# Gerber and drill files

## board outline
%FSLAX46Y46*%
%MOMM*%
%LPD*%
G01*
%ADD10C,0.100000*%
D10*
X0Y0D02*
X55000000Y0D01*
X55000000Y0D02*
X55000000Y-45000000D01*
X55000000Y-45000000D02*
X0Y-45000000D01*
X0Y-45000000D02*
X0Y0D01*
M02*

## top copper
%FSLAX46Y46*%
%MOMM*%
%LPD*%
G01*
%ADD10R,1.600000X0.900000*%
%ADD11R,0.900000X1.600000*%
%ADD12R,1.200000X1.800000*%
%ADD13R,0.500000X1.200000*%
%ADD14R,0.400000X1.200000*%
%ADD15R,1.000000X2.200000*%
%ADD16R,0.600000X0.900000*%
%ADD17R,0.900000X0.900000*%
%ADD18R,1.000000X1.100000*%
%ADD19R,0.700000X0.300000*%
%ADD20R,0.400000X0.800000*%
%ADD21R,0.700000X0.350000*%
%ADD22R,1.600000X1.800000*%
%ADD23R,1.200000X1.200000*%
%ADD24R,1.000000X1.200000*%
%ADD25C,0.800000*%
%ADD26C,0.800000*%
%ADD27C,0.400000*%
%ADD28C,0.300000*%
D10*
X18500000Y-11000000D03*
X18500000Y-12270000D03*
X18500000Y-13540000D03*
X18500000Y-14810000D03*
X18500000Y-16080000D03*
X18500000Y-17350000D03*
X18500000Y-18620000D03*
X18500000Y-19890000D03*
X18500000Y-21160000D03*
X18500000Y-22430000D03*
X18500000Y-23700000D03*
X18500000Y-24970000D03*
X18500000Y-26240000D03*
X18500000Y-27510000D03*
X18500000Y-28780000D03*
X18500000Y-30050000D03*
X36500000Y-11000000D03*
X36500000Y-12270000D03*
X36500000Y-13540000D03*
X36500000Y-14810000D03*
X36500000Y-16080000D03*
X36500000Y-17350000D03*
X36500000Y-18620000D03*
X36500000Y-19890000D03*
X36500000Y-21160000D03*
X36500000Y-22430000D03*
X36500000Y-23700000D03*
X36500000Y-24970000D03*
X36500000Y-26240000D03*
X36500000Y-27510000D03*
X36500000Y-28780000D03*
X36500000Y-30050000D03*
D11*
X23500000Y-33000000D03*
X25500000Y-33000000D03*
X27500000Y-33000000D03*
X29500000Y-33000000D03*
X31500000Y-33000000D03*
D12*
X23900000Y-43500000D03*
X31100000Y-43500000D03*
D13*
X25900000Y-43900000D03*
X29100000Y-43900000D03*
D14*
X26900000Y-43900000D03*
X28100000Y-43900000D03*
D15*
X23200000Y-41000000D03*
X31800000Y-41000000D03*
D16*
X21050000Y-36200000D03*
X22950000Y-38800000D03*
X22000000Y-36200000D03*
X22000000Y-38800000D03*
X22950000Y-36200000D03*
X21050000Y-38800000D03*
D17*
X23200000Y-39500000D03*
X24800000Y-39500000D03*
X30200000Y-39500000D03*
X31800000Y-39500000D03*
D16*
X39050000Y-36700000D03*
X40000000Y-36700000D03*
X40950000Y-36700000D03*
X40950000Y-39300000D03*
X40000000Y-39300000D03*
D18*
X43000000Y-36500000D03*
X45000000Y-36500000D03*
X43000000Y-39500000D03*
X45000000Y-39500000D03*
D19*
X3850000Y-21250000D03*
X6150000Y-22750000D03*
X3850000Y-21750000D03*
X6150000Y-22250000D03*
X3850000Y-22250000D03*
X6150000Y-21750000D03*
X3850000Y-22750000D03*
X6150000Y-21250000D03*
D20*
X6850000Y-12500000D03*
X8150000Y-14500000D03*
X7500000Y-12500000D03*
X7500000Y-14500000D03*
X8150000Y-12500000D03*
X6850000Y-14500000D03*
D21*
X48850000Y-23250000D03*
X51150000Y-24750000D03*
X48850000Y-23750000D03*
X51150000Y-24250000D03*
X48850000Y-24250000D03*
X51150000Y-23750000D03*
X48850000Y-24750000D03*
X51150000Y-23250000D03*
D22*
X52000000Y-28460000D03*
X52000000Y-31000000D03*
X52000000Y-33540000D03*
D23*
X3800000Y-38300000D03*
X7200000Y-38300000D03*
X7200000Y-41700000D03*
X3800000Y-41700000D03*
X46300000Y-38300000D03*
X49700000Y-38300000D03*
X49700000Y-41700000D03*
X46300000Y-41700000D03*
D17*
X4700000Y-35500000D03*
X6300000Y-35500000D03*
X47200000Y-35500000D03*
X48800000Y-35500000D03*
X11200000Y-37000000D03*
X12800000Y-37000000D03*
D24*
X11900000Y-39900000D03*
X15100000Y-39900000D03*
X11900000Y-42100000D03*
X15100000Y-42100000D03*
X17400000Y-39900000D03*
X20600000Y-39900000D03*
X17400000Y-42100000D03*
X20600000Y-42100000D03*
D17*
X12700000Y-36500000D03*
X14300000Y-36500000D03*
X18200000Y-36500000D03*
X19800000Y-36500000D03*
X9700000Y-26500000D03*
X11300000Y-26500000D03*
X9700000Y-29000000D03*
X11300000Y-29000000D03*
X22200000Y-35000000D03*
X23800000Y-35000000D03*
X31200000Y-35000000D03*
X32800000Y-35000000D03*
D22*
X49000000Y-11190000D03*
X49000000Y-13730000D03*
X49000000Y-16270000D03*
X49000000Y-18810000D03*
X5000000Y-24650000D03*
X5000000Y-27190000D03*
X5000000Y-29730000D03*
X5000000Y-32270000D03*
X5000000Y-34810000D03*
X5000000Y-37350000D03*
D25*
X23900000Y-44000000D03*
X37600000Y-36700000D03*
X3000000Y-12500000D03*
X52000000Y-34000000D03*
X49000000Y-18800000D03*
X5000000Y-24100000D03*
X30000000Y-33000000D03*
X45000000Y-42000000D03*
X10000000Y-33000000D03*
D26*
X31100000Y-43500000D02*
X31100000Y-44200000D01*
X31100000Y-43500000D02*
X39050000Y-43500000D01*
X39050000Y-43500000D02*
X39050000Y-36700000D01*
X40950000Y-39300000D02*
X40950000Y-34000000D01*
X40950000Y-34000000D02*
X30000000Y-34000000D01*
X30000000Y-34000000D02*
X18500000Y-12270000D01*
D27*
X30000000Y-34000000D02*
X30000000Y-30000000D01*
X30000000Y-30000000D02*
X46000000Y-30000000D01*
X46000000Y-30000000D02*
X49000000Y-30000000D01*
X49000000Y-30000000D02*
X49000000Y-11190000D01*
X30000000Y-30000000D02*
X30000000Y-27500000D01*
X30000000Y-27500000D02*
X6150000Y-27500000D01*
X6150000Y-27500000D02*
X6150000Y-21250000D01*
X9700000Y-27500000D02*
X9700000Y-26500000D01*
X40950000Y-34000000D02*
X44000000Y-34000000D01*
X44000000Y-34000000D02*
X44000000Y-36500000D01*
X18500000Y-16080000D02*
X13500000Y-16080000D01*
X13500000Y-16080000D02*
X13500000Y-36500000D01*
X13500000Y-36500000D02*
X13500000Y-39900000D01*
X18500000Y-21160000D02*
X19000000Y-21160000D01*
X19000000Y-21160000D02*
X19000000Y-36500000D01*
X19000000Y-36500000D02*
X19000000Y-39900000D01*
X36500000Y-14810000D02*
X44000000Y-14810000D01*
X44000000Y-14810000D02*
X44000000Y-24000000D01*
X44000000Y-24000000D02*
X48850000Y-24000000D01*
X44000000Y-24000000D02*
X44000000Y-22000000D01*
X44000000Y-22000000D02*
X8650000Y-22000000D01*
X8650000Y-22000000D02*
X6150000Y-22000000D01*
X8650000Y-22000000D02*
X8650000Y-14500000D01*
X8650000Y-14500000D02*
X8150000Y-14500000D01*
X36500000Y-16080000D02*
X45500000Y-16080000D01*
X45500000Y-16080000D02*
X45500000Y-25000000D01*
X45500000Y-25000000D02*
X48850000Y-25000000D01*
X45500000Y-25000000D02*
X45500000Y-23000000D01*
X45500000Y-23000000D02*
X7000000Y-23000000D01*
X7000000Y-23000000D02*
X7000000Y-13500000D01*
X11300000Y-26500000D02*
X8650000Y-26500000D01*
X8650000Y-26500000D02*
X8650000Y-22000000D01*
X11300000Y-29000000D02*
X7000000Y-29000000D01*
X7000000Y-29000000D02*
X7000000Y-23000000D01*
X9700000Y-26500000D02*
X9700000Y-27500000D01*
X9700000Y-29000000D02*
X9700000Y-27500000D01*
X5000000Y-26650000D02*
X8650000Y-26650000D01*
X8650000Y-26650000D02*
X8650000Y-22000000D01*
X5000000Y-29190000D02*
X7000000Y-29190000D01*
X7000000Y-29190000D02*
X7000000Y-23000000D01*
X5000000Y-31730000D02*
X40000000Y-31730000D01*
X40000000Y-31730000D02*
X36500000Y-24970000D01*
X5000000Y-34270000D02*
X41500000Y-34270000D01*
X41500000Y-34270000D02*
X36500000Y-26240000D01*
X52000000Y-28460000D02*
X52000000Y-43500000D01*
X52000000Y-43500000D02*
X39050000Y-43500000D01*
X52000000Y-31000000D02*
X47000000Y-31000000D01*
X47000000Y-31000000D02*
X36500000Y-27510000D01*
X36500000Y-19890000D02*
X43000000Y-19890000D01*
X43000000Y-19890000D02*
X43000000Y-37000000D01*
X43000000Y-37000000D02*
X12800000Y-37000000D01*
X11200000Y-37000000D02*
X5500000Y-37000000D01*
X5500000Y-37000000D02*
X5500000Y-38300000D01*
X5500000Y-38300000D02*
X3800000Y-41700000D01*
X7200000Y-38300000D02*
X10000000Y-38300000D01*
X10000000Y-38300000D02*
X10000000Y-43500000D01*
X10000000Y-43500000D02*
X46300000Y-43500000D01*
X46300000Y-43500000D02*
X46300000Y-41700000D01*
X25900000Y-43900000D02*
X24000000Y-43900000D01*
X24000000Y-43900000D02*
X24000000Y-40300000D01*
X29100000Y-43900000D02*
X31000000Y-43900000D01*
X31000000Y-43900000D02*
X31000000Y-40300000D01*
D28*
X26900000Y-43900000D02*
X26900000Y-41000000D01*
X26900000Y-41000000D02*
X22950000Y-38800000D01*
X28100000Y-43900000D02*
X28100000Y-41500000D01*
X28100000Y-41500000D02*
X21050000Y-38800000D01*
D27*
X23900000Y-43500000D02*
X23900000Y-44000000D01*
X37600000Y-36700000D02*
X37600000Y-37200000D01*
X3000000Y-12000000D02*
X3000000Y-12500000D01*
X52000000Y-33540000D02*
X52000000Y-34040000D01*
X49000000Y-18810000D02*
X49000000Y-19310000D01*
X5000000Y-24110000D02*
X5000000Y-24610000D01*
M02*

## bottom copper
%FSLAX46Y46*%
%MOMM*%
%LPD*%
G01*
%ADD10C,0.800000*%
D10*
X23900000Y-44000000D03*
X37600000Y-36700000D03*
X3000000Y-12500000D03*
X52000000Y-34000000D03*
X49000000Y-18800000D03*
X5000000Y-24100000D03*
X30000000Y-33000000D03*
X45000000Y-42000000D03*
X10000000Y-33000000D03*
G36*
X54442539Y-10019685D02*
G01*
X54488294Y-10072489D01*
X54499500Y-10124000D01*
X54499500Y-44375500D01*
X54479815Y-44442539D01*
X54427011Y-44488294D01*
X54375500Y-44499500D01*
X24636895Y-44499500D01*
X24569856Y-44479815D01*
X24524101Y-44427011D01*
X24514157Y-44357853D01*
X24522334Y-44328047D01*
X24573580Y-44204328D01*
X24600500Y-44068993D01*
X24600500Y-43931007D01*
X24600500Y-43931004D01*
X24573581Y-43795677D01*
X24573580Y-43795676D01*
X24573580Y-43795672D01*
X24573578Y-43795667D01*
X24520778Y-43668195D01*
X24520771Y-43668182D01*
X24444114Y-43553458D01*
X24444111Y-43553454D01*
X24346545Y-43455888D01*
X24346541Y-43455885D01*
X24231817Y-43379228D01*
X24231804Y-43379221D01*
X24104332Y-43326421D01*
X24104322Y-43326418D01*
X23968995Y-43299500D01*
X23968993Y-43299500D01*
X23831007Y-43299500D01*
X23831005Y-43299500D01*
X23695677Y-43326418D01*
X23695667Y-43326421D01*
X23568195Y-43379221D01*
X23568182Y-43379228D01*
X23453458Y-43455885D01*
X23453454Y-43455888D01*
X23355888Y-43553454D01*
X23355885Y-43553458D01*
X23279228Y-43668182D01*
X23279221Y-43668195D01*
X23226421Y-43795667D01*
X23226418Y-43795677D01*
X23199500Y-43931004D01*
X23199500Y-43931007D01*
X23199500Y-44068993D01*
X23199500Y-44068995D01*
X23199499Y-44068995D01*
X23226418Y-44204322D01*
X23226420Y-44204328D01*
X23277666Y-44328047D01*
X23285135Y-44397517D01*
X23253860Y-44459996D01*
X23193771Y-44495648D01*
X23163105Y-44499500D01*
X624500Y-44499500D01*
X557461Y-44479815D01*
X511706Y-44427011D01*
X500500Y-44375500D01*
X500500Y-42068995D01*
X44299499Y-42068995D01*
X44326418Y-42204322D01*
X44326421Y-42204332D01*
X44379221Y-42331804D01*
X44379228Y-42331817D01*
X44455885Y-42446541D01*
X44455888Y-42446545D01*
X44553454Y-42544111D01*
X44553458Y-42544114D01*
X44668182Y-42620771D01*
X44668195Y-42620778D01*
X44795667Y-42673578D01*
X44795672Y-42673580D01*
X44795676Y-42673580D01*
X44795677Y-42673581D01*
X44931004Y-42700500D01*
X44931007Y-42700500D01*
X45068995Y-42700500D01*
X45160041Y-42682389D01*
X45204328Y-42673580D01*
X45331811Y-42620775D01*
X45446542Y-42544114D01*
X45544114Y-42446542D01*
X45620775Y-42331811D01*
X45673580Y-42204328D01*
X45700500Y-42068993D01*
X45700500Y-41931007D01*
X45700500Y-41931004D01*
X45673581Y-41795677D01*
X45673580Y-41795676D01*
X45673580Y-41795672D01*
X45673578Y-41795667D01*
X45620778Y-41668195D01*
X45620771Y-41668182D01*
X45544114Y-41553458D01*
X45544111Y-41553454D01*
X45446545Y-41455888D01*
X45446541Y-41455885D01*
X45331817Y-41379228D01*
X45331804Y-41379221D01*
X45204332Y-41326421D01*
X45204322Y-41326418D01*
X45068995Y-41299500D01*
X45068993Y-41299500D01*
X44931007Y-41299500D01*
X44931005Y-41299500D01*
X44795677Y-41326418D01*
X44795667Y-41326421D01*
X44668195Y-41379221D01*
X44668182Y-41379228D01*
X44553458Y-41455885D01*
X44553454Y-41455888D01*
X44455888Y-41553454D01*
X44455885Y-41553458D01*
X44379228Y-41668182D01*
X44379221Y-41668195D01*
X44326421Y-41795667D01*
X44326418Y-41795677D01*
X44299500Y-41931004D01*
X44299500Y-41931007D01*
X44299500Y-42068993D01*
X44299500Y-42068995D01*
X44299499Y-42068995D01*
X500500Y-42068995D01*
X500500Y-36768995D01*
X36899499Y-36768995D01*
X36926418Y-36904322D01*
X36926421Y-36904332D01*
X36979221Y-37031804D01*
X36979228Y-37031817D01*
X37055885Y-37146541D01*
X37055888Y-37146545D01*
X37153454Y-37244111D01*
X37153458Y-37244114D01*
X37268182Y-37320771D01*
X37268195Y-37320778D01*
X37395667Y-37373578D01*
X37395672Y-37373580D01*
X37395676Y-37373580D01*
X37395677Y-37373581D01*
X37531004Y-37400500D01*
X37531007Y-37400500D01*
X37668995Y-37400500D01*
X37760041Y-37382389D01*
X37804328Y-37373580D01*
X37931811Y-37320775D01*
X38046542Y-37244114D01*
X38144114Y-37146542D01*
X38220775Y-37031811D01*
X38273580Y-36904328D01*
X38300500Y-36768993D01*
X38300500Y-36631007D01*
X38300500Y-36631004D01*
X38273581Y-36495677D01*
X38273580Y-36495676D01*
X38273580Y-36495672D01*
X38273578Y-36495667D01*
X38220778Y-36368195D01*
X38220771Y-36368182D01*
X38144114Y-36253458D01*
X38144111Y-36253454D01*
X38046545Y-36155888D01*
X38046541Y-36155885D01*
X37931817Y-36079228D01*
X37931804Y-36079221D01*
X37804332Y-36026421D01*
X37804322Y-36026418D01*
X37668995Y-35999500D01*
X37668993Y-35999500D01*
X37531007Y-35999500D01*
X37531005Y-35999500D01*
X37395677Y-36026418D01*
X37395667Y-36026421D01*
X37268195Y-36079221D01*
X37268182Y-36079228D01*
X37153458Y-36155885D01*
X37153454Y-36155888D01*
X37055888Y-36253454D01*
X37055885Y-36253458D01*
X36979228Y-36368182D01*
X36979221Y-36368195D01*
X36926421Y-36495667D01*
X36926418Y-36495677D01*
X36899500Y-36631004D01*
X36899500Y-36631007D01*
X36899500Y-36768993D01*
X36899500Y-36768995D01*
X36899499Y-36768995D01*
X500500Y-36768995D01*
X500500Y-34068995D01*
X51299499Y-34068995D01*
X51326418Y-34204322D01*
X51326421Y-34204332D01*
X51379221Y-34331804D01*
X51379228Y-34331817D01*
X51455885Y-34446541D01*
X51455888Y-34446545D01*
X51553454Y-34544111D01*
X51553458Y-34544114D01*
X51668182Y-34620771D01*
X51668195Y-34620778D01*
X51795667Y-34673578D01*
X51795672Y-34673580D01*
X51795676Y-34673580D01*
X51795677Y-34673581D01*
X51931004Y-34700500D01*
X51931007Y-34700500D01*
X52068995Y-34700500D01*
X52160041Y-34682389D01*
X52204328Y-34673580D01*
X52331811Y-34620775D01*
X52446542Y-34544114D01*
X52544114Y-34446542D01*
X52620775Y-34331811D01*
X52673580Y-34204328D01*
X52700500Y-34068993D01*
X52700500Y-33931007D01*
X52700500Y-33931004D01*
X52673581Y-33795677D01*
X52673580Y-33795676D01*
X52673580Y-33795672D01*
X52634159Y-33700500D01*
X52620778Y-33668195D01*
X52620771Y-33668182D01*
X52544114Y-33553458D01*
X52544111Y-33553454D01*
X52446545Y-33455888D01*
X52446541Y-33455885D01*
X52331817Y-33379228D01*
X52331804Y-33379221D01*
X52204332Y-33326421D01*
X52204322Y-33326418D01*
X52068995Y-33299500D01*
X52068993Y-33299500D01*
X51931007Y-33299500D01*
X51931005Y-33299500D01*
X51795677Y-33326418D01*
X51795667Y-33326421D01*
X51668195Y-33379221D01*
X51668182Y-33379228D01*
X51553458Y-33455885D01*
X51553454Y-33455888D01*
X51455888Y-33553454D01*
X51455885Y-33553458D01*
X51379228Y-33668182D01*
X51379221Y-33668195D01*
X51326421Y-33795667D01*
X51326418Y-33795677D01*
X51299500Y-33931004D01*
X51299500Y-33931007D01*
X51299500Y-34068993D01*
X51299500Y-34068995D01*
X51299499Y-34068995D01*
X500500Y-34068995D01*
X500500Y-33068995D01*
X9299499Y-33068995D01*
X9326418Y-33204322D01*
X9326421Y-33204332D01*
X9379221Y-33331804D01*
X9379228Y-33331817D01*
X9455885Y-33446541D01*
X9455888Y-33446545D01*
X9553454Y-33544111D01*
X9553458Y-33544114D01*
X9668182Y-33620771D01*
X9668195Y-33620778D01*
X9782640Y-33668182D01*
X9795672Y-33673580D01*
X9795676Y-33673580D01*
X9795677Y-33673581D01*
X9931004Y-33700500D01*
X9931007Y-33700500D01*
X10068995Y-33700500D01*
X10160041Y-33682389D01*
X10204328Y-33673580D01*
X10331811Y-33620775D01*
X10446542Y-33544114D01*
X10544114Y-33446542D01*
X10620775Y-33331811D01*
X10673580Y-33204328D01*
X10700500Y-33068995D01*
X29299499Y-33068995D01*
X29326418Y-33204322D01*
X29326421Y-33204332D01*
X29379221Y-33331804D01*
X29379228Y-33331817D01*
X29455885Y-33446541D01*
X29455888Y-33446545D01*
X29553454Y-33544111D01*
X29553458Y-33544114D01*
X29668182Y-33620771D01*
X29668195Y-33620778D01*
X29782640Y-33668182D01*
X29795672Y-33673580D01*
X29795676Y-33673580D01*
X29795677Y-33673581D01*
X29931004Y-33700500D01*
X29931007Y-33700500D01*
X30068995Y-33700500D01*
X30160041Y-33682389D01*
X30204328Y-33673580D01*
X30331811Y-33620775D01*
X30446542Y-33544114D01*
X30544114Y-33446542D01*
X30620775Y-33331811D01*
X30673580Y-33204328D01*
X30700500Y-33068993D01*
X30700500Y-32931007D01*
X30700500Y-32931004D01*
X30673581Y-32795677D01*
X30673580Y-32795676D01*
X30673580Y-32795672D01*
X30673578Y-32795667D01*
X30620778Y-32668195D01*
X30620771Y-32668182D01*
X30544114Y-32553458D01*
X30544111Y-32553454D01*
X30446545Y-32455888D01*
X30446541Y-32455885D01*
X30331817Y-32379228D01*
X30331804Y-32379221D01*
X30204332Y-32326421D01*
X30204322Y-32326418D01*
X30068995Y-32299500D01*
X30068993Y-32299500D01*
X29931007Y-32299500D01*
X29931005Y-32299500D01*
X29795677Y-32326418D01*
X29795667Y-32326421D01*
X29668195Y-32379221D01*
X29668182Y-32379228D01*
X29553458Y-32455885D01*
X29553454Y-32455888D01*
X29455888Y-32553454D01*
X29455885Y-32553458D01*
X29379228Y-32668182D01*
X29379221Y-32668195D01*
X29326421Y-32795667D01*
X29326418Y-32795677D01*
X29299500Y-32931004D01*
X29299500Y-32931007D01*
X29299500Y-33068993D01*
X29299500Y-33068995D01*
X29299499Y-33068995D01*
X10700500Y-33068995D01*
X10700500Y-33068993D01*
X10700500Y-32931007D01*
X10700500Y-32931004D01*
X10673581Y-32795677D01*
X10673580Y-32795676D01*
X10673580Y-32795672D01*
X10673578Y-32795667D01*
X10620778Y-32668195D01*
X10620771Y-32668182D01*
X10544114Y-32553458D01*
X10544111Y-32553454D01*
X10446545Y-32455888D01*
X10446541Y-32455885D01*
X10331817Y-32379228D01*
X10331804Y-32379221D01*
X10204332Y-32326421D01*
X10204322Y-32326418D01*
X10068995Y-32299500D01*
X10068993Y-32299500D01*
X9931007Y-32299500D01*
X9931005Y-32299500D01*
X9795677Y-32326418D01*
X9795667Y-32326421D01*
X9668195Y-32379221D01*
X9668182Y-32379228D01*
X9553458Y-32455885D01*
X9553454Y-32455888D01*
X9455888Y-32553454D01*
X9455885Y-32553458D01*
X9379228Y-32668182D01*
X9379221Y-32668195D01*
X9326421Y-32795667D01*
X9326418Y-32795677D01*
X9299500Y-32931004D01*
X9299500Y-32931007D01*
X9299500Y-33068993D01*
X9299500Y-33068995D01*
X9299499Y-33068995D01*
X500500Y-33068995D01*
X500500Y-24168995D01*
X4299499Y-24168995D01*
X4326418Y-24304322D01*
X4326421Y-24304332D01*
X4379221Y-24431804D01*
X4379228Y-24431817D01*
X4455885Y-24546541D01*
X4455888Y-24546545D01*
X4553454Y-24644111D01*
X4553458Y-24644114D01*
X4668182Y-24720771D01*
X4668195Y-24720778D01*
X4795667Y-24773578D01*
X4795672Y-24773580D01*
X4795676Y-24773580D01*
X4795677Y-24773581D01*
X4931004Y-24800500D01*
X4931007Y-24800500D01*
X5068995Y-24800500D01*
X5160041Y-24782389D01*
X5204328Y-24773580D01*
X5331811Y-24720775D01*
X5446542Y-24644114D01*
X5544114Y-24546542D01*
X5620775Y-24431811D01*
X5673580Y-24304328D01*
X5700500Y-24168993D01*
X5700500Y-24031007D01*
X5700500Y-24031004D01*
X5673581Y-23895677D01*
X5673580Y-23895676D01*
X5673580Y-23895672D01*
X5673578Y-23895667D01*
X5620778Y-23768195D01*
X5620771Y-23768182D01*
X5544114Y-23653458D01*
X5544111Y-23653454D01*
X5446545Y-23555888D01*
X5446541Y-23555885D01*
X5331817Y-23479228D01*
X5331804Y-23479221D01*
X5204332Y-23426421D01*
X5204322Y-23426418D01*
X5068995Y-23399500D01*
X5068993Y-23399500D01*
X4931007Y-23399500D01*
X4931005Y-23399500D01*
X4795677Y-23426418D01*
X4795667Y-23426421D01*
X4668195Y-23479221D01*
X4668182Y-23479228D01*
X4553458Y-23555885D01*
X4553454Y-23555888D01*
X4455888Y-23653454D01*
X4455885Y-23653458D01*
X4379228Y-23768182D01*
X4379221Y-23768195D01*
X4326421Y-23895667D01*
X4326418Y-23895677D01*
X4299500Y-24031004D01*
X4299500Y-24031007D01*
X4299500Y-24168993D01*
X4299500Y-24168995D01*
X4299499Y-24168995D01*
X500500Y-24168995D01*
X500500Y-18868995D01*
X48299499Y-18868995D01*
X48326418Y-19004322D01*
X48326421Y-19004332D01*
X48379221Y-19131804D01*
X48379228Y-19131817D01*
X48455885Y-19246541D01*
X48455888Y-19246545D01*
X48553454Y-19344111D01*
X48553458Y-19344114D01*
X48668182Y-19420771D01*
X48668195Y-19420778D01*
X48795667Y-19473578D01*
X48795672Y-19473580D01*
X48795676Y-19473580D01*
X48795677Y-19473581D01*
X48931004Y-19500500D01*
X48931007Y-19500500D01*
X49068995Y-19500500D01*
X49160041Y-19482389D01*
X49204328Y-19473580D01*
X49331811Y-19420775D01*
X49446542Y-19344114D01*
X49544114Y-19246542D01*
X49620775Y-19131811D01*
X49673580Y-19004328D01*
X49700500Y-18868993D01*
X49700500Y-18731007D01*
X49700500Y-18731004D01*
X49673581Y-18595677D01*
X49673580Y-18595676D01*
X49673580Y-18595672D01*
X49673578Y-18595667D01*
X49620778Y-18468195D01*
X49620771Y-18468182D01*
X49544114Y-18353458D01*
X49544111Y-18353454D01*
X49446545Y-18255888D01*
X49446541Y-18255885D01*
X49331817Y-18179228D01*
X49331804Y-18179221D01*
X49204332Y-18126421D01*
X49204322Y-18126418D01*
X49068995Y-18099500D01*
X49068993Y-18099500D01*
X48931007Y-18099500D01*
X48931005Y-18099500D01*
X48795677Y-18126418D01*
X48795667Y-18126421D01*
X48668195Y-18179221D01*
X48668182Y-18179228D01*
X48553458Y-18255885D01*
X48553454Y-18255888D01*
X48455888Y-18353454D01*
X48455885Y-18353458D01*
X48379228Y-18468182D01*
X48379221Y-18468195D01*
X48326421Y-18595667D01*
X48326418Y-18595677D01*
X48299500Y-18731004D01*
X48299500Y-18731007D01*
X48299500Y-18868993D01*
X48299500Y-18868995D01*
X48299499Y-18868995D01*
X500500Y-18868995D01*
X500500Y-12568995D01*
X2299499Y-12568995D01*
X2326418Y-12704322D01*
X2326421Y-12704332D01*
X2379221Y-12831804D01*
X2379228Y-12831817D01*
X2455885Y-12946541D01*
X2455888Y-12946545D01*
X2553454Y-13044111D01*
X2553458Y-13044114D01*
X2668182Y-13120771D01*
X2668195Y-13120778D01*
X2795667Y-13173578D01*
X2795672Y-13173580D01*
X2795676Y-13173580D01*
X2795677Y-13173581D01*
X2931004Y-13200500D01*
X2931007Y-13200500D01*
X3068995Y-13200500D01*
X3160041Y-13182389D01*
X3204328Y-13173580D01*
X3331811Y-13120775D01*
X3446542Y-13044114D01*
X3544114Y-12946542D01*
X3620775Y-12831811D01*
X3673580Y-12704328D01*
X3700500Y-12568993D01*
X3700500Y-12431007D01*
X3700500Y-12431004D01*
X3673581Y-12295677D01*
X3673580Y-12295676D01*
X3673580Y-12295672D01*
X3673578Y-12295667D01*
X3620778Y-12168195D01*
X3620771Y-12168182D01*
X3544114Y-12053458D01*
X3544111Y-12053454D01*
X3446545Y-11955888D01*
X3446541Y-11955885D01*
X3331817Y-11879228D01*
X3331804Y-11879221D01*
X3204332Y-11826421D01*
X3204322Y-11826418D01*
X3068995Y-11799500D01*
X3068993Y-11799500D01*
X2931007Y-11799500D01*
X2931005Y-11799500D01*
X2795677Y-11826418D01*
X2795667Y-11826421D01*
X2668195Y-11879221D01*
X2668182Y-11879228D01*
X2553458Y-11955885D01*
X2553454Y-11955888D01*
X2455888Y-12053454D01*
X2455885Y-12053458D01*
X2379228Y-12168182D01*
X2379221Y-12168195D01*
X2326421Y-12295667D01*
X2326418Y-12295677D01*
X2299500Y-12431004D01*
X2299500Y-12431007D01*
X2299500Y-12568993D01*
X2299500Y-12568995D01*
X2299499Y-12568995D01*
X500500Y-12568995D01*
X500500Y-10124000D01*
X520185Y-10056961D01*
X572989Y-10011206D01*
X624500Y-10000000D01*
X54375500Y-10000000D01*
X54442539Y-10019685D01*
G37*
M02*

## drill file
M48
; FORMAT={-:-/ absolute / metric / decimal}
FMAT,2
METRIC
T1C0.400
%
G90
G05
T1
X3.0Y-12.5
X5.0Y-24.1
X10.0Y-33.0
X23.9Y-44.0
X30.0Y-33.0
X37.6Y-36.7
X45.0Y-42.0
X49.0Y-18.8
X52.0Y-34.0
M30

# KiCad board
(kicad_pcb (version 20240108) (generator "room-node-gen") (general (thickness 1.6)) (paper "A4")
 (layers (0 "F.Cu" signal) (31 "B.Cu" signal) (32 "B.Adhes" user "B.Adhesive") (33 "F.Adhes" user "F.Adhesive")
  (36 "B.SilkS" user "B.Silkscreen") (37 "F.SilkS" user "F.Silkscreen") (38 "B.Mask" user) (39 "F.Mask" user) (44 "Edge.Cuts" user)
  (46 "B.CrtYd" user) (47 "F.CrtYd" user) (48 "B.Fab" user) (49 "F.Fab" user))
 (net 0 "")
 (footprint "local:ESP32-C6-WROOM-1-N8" (layer "F.Cu") (at 27.500 22.000 0)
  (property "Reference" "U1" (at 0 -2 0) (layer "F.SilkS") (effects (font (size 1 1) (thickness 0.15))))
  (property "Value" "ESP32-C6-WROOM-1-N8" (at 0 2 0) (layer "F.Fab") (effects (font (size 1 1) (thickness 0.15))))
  (pad "1" smd rect (at -9.000 -11.000) (size 1.600 0.900) (layers "F.Cu"))
  (pad "2" smd rect (at -9.000 -9.730) (size 1.600 0.900) (layers "F.Cu"))
  (pad "3" smd rect (at -9.000 -8.460) (size 1.600 0.900) (layers "F.Cu"))
  (pad "4" smd rect (at -9.000 -7.190) (size 1.600 0.900) (layers "F.Cu"))
  (pad "5" smd rect (at -9.000 -5.920) (size 1.600 0.900) (layers "F.Cu"))
  (pad "6" smd rect (at -9.000 -4.650) (size 1.600 0.900) (layers "F.Cu"))
  (pad "7" smd rect (at -9.000 -3.380) (size 1.600 0.900) (layers "F.Cu"))
  (pad "8" smd rect (at -9.000 -2.110) (size 1.600 0.900) (layers "F.Cu"))
  (pad "9" smd rect (at -9.000 -0.840) (size 1.600 0.900) (layers "F.Cu"))
  (pad "10" smd rect (at -9.000 0.430) (size 1.600 0.900) (layers "F.Cu"))
  (pad "11" smd rect (at -9.000 1.700) (size 1.600 0.900) (layers "F.Cu"))
  (pad "12" smd rect (at -9.000 2.970) (size 1.600 0.900) (layers "F.Cu"))
  (pad "13" smd rect (at -9.000 4.240) (size 1.600 0.900) (layers "F.Cu"))
  (pad "14" smd rect (at -9.000 5.510) (size 1.600 0.900) (layers "F.Cu"))
  (pad "15" smd rect (at -9.000 6.780) (size 1.600 0.900) (layers "F.Cu"))
  (pad "16" smd rect (at -9.000 8.050) (size 1.600 0.900) (layers "F.Cu"))
  (pad "17" smd rect (at 9.000 -11.000) (size 1.600 0.900) (layers "F.Cu"))
  (pad "18" smd rect (at 9.000 -9.730) (size 1.600 0.900) (layers "F.Cu"))
  (pad "19" smd rect (at 9.000 -8.460) (size 1.600 0.900) (layers "F.Cu"))
  (pad "20" smd rect (at 9.000 -7.190) (size 1.600 0.900) (layers "F.Cu"))
  (pad "21" smd rect (at 9.000 -5.920) (size 1.600 0.900) (layers "F.Cu"))
  (pad "22" smd rect (at 9.000 -4.650) (size 1.600 0.900) (layers "F.Cu"))
  (pad "23" smd rect (at 9.000 -3.380) (size 1.600 0.900) (layers "F.Cu"))
  (pad "24" smd rect (at 9.000 -2.110) (size 1.600 0.900) (layers "F.Cu"))
  (pad "25" smd rect (at 9.000 -0.840) (size 1.600 0.900) (layers "F.Cu"))
  (pad "26" smd rect (at 9.000 0.430) (size 1.600 0.900) (layers "F.Cu"))
  (pad "27" smd rect (at 9.000 1.700) (size 1.600 0.900) (layers "F.Cu"))
  (pad "28" smd rect (at 9.000 2.970) (size 1.600 0.900) (layers "F.Cu"))
  (pad "29" smd rect (at 9.000 4.240) (size 1.600 0.900) (layers "F.Cu"))
  (pad "30" smd rect (at 9.000 5.510) (size 1.600 0.900) (layers "F.Cu"))
  (pad "31" smd rect (at 9.000 6.780) (size 1.600 0.900) (layers "F.Cu"))
  (pad "32" smd rect (at 9.000 8.050) (size 1.600 0.900) (layers "F.Cu"))
  (pad "33" smd rect (at -4.000 11.000) (size 0.900 1.600) (layers "F.Cu"))
  (pad "34" smd rect (at -2.000 11.000) (size 0.900 1.600) (layers "F.Cu"))
  (pad "35" smd rect (at 0.000 11.000) (size 0.900 1.600) (layers "F.Cu"))
  (pad "36" smd rect (at 2.000 11.000) (size 0.900 1.600) (layers "F.Cu"))
  (pad "37" smd rect (at 4.000 11.000) (size 0.900 1.600) (layers "F.Cu")))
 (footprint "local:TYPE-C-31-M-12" (layer "F.Cu") (at 27.500 42.000 0)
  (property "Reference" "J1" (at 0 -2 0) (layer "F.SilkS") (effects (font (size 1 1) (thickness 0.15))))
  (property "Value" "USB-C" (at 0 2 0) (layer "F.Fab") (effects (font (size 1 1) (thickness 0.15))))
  (pad "GND" smd rect (at -3.600 1.500) (size 1.200 1.800) (layers "F.Cu"))
  (pad "VBUS" smd rect (at 3.600 1.500) (size 1.200 1.800) (layers "F.Cu"))
  (pad "CC1" smd rect (at -1.600 1.900) (size 0.500 1.200) (layers "F.Cu"))
  (pad "CC2" smd rect (at 1.600 1.900) (size 0.500 1.200) (layers "F.Cu"))
  (pad "DM" smd rect (at -0.600 1.900) (size 0.400 1.200) (layers "F.Cu"))
  (pad "DP" smd rect (at 0.600 1.900) (size 0.400 1.200) (layers "F.Cu"))
  (pad "SH1" smd rect (at -4.300 -1.000) (size 1.000 2.200) (layers "F.Cu"))
  (pad "SH2" smd rect (at 4.300 -1.000) (size 1.000 2.200) (layers "F.Cu")))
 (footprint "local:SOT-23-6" (layer "F.Cu") (at 22.000 37.500 0)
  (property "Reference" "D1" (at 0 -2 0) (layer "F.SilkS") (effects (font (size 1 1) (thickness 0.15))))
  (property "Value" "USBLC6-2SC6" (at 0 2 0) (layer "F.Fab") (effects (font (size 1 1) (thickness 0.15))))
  (pad "1" smd rect (at -0.950 -1.300) (size 0.600 0.900) (layers "F.Cu"))
  (pad "4" smd rect (at 0.950 1.300) (size 0.600 0.900) (layers "F.Cu"))
  (pad "2" smd rect (at 0.000 -1.300) (size 0.600 0.900) (layers "F.Cu"))
  (pad "5" smd rect (at 0.000 1.300) (size 0.600 0.900) (layers "F.Cu"))
  (pad "3" smd rect (at 0.950 -1.300) (size 0.600 0.900) (layers "F.Cu"))
  (pad "6" smd rect (at -0.950 1.300) (size 0.600 0.900) (layers "F.Cu")))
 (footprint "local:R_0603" (layer "F.Cu") (at 24.000 39.500 0)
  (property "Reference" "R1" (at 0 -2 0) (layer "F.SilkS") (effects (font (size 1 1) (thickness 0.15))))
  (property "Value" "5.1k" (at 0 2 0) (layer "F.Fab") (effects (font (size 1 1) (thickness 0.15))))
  (pad "1" smd rect (at -0.800 0.000) (size 0.900 0.900) (layers "F.Cu"))
  (pad "2" smd rect (at 0.800 0.000) (size 0.900 0.900) (layers "F.Cu")))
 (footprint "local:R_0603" (layer "F.Cu") (at 31.000 39.500 0)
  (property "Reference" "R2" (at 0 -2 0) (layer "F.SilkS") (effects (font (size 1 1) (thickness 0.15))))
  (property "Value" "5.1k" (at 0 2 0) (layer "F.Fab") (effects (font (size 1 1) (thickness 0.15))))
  (pad "1" smd rect (at -0.800 0.000) (size 0.900 0.900) (layers "F.Cu"))
  (pad "2" smd rect (at 0.800 0.000) (size 0.900 0.900) (layers "F.Cu")))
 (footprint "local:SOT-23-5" (layer "F.Cu") (at 40.000 38.000 0)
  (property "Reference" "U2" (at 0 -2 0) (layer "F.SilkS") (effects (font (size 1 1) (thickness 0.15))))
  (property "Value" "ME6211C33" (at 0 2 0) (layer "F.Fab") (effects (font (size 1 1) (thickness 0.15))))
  (pad "1" smd rect (at -0.950 -1.300) (size 0.600 0.900) (layers "F.Cu"))
  (pad "2" smd rect (at 0.000 -1.300) (size 0.600 0.900) (layers "F.Cu"))
  (pad "3" smd rect (at 0.950 -1.300) (size 0.600 0.900) (layers "F.Cu"))
  (pad "4" smd rect (at 0.950 1.300) (size 0.600 0.900) (layers "F.Cu"))
  (pad "5" smd rect (at 0.000 1.300) (size 0.600 0.900) (layers "F.Cu")))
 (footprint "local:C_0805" (layer "F.Cu") (at 44.000 36.500 0)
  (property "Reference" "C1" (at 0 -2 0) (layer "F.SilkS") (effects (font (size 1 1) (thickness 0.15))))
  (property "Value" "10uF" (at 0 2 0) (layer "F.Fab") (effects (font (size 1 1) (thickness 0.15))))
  (pad "1" smd rect (at -1.000 0.000) (size 1.000 1.100) (layers "F.Cu"))
  (pad "2" smd rect (at 1.000 0.000) (size 1.000 1.100) (layers "F.Cu")))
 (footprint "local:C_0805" (layer "F.Cu") (at 44.000 39.500 0)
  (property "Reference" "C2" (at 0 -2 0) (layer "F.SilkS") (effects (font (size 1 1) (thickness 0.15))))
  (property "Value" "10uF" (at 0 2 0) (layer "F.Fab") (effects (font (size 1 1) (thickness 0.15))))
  (pad "1" smd rect (at -1.000 0.000) (size 1.000 1.100) (layers "F.Cu"))
  (pad "2" smd rect (at 1.000 0.000) (size 1.000 1.100) (layers "F.Cu")))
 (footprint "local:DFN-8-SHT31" (layer "F.Cu") (at 5.000 22.000 0)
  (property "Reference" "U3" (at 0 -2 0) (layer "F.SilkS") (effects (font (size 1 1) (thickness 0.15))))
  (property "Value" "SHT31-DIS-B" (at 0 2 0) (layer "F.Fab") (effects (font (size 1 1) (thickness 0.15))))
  (pad "1" smd rect (at -1.150 -0.750) (size 0.700 0.300) (layers "F.Cu"))
  (pad "5" smd rect (at 1.150 0.750) (size 0.700 0.300) (layers "F.Cu"))
  (pad "2" smd rect (at -1.150 -0.250) (size 0.700 0.300) (layers "F.Cu"))
  (pad "6" smd rect (at 1.150 0.250) (size 0.700 0.300) (layers "F.Cu"))
  (pad "3" smd rect (at -1.150 0.250) (size 0.700 0.300) (layers "F.Cu"))
  (pad "7" smd rect (at 1.150 -0.250) (size 0.700 0.300) (layers "F.Cu"))
  (pad "4" smd rect (at -1.150 0.750) (size 0.700 0.300) (layers "F.Cu"))
  (pad "8" smd rect (at 1.150 -0.750) (size 0.700 0.300) (layers "F.Cu")))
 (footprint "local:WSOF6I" (layer "F.Cu") (at 7.500 13.500 0)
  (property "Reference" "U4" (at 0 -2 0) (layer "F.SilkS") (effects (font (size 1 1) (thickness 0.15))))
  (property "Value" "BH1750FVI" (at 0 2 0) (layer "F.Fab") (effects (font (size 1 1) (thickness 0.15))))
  (pad "1" smd rect (at -0.650 -1.000) (size 0.400 0.800) (layers "F.Cu"))
  (pad "4" smd rect (at 0.650 1.000) (size 0.400 0.800) (layers "F.Cu"))
  (pad "2" smd rect (at 0.000 -1.000) (size 0.400 0.800) (layers "F.Cu"))
  (pad "5" smd rect (at 0.000 1.000) (size 0.400 0.800) (layers "F.Cu"))
  (pad "3" smd rect (at 0.650 -1.000) (size 0.400 0.800) (layers "F.Cu"))
  (pad "6" smd rect (at -0.650 1.000) (size 0.400 0.800) (layers "F.Cu")))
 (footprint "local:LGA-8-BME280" (layer "F.Cu") (at 50.000 24.000 0)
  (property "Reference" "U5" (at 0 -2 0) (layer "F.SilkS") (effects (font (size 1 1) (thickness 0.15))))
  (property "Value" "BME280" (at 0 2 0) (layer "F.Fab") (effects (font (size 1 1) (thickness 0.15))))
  (pad "1" smd rect (at -1.150 -0.750) (size 0.700 0.350) (layers "F.Cu"))
  (pad "5" smd rect (at 1.150 0.750) (size 0.700 0.350) (layers "F.Cu"))
  (pad "2" smd rect (at -1.150 -0.250) (size 0.700 0.350) (layers "F.Cu"))
  (pad "6" smd rect (at 1.150 0.250) (size 0.700 0.350) (layers "F.Cu"))
  (pad "3" smd rect (at -1.150 0.250) (size 0.700 0.350) (layers "F.Cu"))
  (pad "7" smd rect (at 1.150 -0.250) (size 0.700 0.350) (layers "F.Cu"))
  (pad "4" smd rect (at -1.150 0.750) (size 0.700 0.350) (layers "F.Cu"))
  (pad "8" smd rect (at 1.150 -0.750) (size 0.700 0.350) (layers "F.Cu")))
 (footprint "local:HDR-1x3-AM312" (layer "F.Cu") (at 52.000 31.000 0)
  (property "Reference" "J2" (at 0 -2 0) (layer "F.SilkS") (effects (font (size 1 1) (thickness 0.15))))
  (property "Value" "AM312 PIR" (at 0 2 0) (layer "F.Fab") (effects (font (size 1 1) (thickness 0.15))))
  (pad "VIN" smd rect (at 0.000 -2.540) (size 1.600 1.800) (layers "F.Cu"))
  (pad "OUT" smd rect (at 0.000 0.000) (size 1.600 1.800) (layers "F.Cu"))
  (pad "GND" smd rect (at 0.000 2.540) (size 1.600 1.800) (layers "F.Cu")))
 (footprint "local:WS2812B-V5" (layer "F.Cu") (at 5.500 40.000 0)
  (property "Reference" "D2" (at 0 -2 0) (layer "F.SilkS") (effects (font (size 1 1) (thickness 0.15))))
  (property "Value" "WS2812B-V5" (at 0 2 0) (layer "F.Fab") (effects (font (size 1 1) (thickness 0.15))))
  (pad "VDD" smd rect (at -1.700 -1.700) (size 1.200 1.200) (layers "F.Cu"))
  (pad "DOUT" smd rect (at 1.700 -1.700) (size 1.200 1.200) (layers "F.Cu"))
  (pad "VSS" smd rect (at 1.700 1.700) (size 1.200 1.200) (layers "F.Cu"))
  (pad "DIN" smd rect (at -1.700 1.700) (size 1.200 1.200) (layers "F.Cu")))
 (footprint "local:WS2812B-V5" (layer "F.Cu") (at 48.000 40.000 0)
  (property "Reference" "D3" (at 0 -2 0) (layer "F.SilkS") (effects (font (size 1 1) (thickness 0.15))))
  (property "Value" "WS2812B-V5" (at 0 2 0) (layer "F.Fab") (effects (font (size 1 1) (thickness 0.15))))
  (pad "VDD" smd rect (at -1.700 -1.700) (size 1.200 1.200) (layers "F.Cu"))
  (pad "DOUT" smd rect (at 1.700 -1.700) (size 1.200 1.200) (layers "F.Cu"))
  (pad "VSS" smd rect (at 1.700 1.700) (size 1.200 1.200) (layers "F.Cu"))
  (pad "DIN" smd rect (at -1.700 1.700) (size 1.200 1.200) (layers "F.Cu")))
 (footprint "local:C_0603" (layer "F.Cu") (at 5.500 35.500 0)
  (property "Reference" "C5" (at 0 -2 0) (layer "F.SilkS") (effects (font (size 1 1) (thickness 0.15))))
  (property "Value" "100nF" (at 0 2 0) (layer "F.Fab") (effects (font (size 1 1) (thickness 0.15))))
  (pad "1" smd rect (at -0.800 0.000) (size 0.900 0.900) (layers "F.Cu"))
  (pad "2" smd rect (at 0.800 0.000) (size 0.900 0.900) (layers "F.Cu")))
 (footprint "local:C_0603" (layer "F.Cu") (at 48.000 35.500 0)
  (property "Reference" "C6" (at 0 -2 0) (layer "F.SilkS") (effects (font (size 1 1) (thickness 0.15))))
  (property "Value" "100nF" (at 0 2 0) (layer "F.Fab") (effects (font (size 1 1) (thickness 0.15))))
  (pad "1" smd rect (at -0.800 0.000) (size 0.900 0.900) (layers "F.Cu"))
  (pad "2" smd rect (at 0.800 0.000) (size 0.900 0.900) (layers "F.Cu")))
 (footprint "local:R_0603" (layer "F.Cu") (at 12.000 37.000 0)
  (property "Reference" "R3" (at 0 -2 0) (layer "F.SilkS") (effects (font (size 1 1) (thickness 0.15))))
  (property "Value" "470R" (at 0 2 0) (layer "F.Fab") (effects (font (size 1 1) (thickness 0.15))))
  (pad "1" smd rect (at -0.800 0.000) (size 0.900 0.900) (layers "F.Cu"))
  (pad "2" smd rect (at 0.800 0.000) (size 0.900 0.900) (layers "F.Cu")))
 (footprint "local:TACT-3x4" (layer "F.Cu") (at 13.500 41.000 0)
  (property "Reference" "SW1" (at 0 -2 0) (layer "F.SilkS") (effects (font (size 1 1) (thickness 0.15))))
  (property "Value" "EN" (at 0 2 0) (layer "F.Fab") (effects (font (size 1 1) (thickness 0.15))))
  (pad "1" smd rect (at -1.600 -1.100) (size 1.000 1.200) (layers "F.Cu"))
  (pad "2" smd rect (at 1.600 -1.100) (size 1.000 1.200) (layers "F.Cu"))
  (pad "3" smd rect (at -1.600 1.100) (size 1.000 1.200) (layers "F.Cu"))
  (pad "4" smd rect (at 1.600 1.100) (size 1.000 1.200) (layers "F.Cu")))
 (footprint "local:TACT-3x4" (layer "F.Cu") (at 19.000 41.000 0)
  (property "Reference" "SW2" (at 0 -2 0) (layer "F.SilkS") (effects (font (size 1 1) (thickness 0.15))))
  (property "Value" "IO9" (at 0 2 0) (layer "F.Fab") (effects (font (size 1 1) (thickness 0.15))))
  (pad "1" smd rect (at -1.600 -1.100) (size 1.000 1.200) (layers "F.Cu"))
  (pad "2" smd rect (at 1.600 -1.100) (size 1.000 1.200) (layers "F.Cu"))
  (pad "3" smd rect (at -1.600 1.100) (size 1.000 1.200) (layers "F.Cu"))
  (pad "4" smd rect (at 1.600 1.100) (size 1.000 1.200) (layers "F.Cu")))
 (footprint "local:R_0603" (layer "F.Cu") (at 13.500 36.500 0)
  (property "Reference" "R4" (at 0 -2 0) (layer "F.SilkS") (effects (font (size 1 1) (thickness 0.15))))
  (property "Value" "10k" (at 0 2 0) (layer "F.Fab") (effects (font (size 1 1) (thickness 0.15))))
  (pad "1" smd rect (at -0.800 0.000) (size 0.900 0.900) (layers "F.Cu"))
  (pad "2" smd rect (at 0.800 0.000) (size 0.900 0.900) (layers "F.Cu")))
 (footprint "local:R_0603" (layer "F.Cu") (at 19.000 36.500 0)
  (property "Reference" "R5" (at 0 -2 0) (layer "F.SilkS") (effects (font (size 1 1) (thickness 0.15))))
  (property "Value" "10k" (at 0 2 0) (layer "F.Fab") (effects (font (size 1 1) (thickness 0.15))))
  (pad "1" smd rect (at -0.800 0.000) (size 0.900 0.900) (layers "F.Cu"))
  (pad "2" smd rect (at 0.800 0.000) (size 0.900 0.900) (layers "F.Cu")))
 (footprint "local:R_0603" (layer "F.Cu") (at 10.500 26.500 0)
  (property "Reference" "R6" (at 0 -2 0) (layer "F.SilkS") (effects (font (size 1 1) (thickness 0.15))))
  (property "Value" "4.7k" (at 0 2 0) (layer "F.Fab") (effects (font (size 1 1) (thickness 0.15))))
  (pad "1" smd rect (at -0.800 0.000) (size 0.900 0.900) (layers "F.Cu"))
  (pad "2" smd rect (at 0.800 0.000) (size 0.900 0.900) (layers "F.Cu")))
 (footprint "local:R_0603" (layer "F.Cu") (at 10.500 29.000 0)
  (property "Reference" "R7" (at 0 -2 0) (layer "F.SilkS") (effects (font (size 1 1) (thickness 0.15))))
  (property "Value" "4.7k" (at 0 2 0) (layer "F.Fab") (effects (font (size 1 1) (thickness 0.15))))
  (pad "1" smd rect (at -0.800 0.000) (size 0.900 0.900) (layers "F.Cu"))
  (pad "2" smd rect (at 0.800 0.000) (size 0.900 0.900) (layers "F.Cu")))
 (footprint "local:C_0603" (layer "F.Cu") (at 23.000 35.000 0)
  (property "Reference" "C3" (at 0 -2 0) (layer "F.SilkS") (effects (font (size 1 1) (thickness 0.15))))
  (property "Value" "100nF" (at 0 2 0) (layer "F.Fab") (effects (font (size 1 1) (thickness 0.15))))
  (pad "1" smd rect (at -0.800 0.000) (size 0.900 0.900) (layers "F.Cu"))
  (pad "2" smd rect (at 0.800 0.000) (size 0.900 0.900) (layers "F.Cu")))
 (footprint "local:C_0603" (layer "F.Cu") (at 32.000 35.000 0)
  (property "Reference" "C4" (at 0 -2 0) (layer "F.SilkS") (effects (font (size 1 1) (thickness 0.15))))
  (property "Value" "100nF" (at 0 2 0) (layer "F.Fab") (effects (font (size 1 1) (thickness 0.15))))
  (pad "1" smd rect (at -0.800 0.000) (size 0.900 0.900) (layers "F.Cu"))
  (pad "2" smd rect (at 0.800 0.000) (size 0.900 0.900) (layers "F.Cu")))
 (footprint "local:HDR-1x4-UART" (layer "F.Cu") (at 49.000 15.000 0)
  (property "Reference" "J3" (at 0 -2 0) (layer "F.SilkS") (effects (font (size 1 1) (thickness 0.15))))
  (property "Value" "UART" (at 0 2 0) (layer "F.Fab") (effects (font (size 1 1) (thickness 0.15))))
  (pad "3V3" smd rect (at 0.000 -3.810) (size 1.600 1.800) (layers "F.Cu"))
  (pad "TX" smd rect (at 0.000 -1.270) (size 1.600 1.800) (layers "F.Cu"))
  (pad "RX" smd rect (at 0.000 1.270) (size 1.600 1.800) (layers "F.Cu"))
  (pad "GND" smd rect (at 0.000 3.810) (size 1.600 1.800) (layers "F.Cu")))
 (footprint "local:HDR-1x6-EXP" (layer "F.Cu") (at 5.000 31.000 0)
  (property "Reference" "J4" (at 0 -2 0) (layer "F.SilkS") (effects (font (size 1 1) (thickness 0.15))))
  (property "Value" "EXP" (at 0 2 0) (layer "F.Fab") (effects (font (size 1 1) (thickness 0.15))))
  (pad "3V3" smd rect (at 0.000 -6.350) (size 1.600 1.800) (layers "F.Cu"))
  (pad "GND" smd rect (at 0.000 -3.810) (size 1.600 1.800) (layers "F.Cu"))
  (pad "SDA" smd rect (at 0.000 -1.270) (size 1.600 1.800) (layers "F.Cu"))
  (pad "SCL" smd rect (at 0.000 1.270) (size 1.600 1.800) (layers "F.Cu"))
  (pad "IO20" smd rect (at 0.000 3.810) (size 1.600 1.800) (layers "F.Cu"))
  (pad "IO21" smd rect (at 0.000 6.350) (size 1.600 1.800) (layers "F.Cu")))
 (gr_line (start 0.000 0.000) (end 55.000 0.000) (stroke (width 0.1) (type solid)) (layer "Edge.Cuts"))
 (gr_line (start 55.000 0.000) (end 55.000 45.000) (stroke (width 0.1) (type solid)) (layer "Edge.Cuts"))
 (gr_line (start 55.000 45.000) (end 0.000 45.000) (stroke (width 0.1) (type solid)) (layer "Edge.Cuts"))
 (gr_line (start 0.000 45.000) (end 0.000 0.000) (stroke (width 0.1) (type solid)) (layer "Edge.Cuts"))
 (segment (start 31.100 43.500) (end 31.100 44.200) (width 0.8) (layer "F.Cu") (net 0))
 (segment (start 31.100 43.500) (end 39.050 43.500) (width 0.8) (layer "F.Cu") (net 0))
 (segment (start 39.050 43.500) (end 39.050 36.700) (width 0.8) (layer "F.Cu") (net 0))
 (segment (start 40.950 39.300) (end 40.950 34.000) (width 0.8) (layer "F.Cu") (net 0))
 (segment (start 40.950 34.000) (end 30.000 34.000) (width 0.8) (layer "F.Cu") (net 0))
 (segment (start 30.000 34.000) (end 18.500 12.270) (width 0.8) (layer "F.Cu") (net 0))
 (segment (start 30.000 34.000) (end 30.000 30.000) (width 0.4) (layer "F.Cu") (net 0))
 (segment (start 30.000 30.000) (end 46.000 30.000) (width 0.4) (layer "F.Cu") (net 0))
 (segment (start 46.000 30.000) (end 49.000 30.000) (width 0.4) (layer "F.Cu") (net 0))
 (segment (start 49.000 30.000) (end 49.000 11.190) (width 0.4) (layer "F.Cu") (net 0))
 (segment (start 30.000 30.000) (end 30.000 27.500) (width 0.4) (layer "F.Cu") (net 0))
 (segment (start 30.000 27.500) (end 6.150 27.500) (width 0.4) (layer "F.Cu") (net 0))
 (segment (start 6.150 27.500) (end 6.150 21.250) (width 0.4) (layer "F.Cu") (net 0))
 (segment (start 9.700 27.500) (end 9.700 26.500) (width 0.4) (layer "F.Cu") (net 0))
 (segment (start 40.950 34.000) (end 44.000 34.000) (width 0.4) (layer "F.Cu") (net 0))
 (segment (start 44.000 34.000) (end 44.000 36.500) (width 0.4) (layer "F.Cu") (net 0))
 (segment (start 18.500 16.080) (end 13.500 16.080) (width 0.4) (layer "F.Cu") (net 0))
 (segment (start 13.500 16.080) (end 13.500 36.500) (width 0.4) (layer "F.Cu") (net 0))
 (segment (start 13.500 36.500) (end 13.500 39.900) (width 0.4) (layer "F.Cu") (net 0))
 (segment (start 18.500 21.160) (end 19.000 21.160) (width 0.4) (layer "F.Cu") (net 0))
 (segment (start 19.000 21.160) (end 19.000 36.500) (width 0.4) (layer "F.Cu") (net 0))
 (segment (start 19.000 36.500) (end 19.000 39.900) (width 0.4) (layer "F.Cu") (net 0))
 (segment (start 36.500 14.810) (end 44.000 14.810) (width 0.4) (layer "F.Cu") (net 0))
 (segment (start 44.000 14.810) (end 44.000 24.000) (width 0.4) (layer "F.Cu") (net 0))
 (segment (start 44.000 24.000) (end 48.850 24.000) (width 0.4) (layer "F.Cu") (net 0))
 (segment (start 44.000 24.000) (end 44.000 22.000) (width 0.4) (layer "F.Cu") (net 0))
 (segment (start 44.000 22.000) (end 8.650 22.000) (width 0.4) (layer "F.Cu") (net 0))
 (segment (start 8.650 22.000) (end 6.150 22.000) (width 0.4) (layer "F.Cu") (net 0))
 (segment (start 8.650 22.000) (end 8.650 14.500) (width 0.4) (layer "F.Cu") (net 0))
 (segment (start 8.650 14.500) (end 8.150 14.500) (width 0.4) (layer "F.Cu") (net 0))
 (segment (start 36.500 16.080) (end 45.500 16.080) (width 0.4) (layer "F.Cu") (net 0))
 (segment (start 45.500 16.080) (end 45.500 25.000) (width 0.4) (layer "F.Cu") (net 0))
 (segment (start 45.500 25.000) (end 48.850 25.000) (width 0.4) (layer "F.Cu") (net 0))
 (segment (start 45.500 25.000) (end 45.500 23.000) (width 0.4) (layer "F.Cu") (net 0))
 (segment (start 45.500 23.000) (end 7.000 23.000) (width 0.4) (layer "F.Cu") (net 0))
 (segment (start 7.000 23.000) (end 7.000 13.500) (width 0.4) (layer "F.Cu") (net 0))
 (segment (start 11.300 26.500) (end 8.650 26.500) (width 0.4) (layer "F.Cu") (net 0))
 (segment (start 8.650 26.500) (end 8.650 22.000) (width 0.4) (layer "F.Cu") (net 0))
 (segment (start 11.300 29.000) (end 7.000 29.000) (width 0.4) (layer "F.Cu") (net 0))
 (segment (start 7.000 29.000) (end 7.000 23.000) (width 0.4) (layer "F.Cu") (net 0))
 (segment (start 9.700 26.500) (end 9.700 27.500) (width 0.4) (layer "F.Cu") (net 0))
 (segment (start 9.700 29.000) (end 9.700 27.500) (width 0.4) (layer "F.Cu") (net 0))
 (segment (start 5.000 26.650) (end 8.650 26.650) (width 0.4) (layer "F.Cu") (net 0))
 (segment (start 8.650 26.650) (end 8.650 22.000) (width 0.4) (layer "F.Cu") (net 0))
 (segment (start 5.000 29.190) (end 7.000 29.190) (width 0.4) (layer "F.Cu") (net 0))
 (segment (start 7.000 29.190) (end 7.000 23.000) (width 0.4) (layer "F.Cu") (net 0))
 (segment (start 5.000 31.730) (end 40.000 31.730) (width 0.4) (layer "F.Cu") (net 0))
 (segment (start 40.000 31.730) (end 36.500 24.970) (width 0.4) (layer "F.Cu") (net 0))
 (segment (start 5.000 34.270) (end 41.500 34.270) (width 0.4) (layer "F.Cu") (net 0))
 (segment (start 41.500 34.270) (end 36.500 26.240) (width 0.4) (layer "F.Cu") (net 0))
 (segment (start 52.000 28.460) (end 52.000 43.500) (width 0.4) (layer "F.Cu") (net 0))
 (segment (start 52.000 43.500) (end 39.050 43.500) (width 0.4) (layer "F.Cu") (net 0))
 (segment (start 52.000 31.000) (end 47.000 31.000) (width 0.4) (layer "F.Cu") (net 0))
 (segment (start 47.000 31.000) (end 36.500 27.510) (width 0.4) (layer "F.Cu") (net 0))
 (segment (start 36.500 19.890) (end 43.000 19.890) (width 0.4) (layer "F.Cu") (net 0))
 (segment (start 43.000 19.890) (end 43.000 37.000) (width 0.4) (layer "F.Cu") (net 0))
 (segment (start 43.000 37.000) (end 12.800 37.000) (width 0.4) (layer "F.Cu") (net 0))
 (segment (start 11.200 37.000) (end 5.500 37.000) (width 0.4) (layer "F.Cu") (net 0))
 (segment (start 5.500 37.000) (end 5.500 38.300) (width 0.4) (layer "F.Cu") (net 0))
 (segment (start 5.500 38.300) (end 3.800 41.700) (width 0.4) (layer "F.Cu") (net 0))
 (segment (start 7.200 38.300) (end 10.000 38.300) (width 0.4) (layer "F.Cu") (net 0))
 (segment (start 10.000 38.300) (end 10.000 43.500) (width 0.4) (layer "F.Cu") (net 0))
 (segment (start 10.000 43.500) (end 46.300 43.500) (width 0.4) (layer "F.Cu") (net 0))
 (segment (start 46.300 43.500) (end 46.300 41.700) (width 0.4) (layer "F.Cu") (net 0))
 (segment (start 25.900 43.900) (end 24.000 43.900) (width 0.4) (layer "F.Cu") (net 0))
 (segment (start 24.000 43.900) (end 24.000 40.300) (width 0.4) (layer "F.Cu") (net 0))
 (segment (start 29.100 43.900) (end 31.000 43.900) (width 0.4) (layer "F.Cu") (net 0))
 (segment (start 31.000 43.900) (end 31.000 40.300) (width 0.4) (layer "F.Cu") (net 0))
 (segment (start 26.900 43.900) (end 26.900 41.000) (width 0.3) (layer "F.Cu") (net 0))
 (segment (start 26.900 41.000) (end 22.950 38.800) (width 0.3) (layer "F.Cu") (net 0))
 (segment (start 28.100 43.900) (end 28.100 41.500) (width 0.3) (layer "F.Cu") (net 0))
 (segment (start 28.100 41.500) (end 21.050 38.800) (width 0.3) (layer "F.Cu") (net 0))
 (segment (start 23.900 43.500) (end 23.900 44.000) (width 0.4) (layer "F.Cu") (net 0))
 (segment (start 37.600 36.700) (end 37.600 37.200) (width 0.4) (layer "F.Cu") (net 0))
 (segment (start 3.000 12.000) (end 3.000 12.500) (width 0.4) (layer "F.Cu") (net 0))
 (segment (start 52.000 33.540) (end 52.000 34.040) (width 0.4) (layer "F.Cu") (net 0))
 (segment (start 49.000 18.810) (end 49.000 19.310) (width 0.4) (layer "F.Cu") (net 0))
 (segment (start 5.000 24.110) (end 5.000 24.610) (width 0.4) (layer "F.Cu") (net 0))
 (via (at 23.900 44.000) (size 0.8) (drill 0.4) (layers "F.Cu" "B.Cu") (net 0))
 (via (at 37.600 36.700) (size 0.8) (drill 0.4) (layers "F.Cu" "B.Cu") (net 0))
 (via (at 3.000 12.500) (size 0.8) (drill 0.4) (layers "F.Cu" "B.Cu") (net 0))
 (via (at 52.000 34.000) (size 0.8) (drill 0.4) (layers "F.Cu" "B.Cu") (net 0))
 (via (at 49.000 18.800) (size 0.8) (drill 0.4) (layers "F.Cu" "B.Cu") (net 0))
 (via (at 5.000 24.100) (size 0.8) (drill 0.4) (layers "F.Cu" "B.Cu") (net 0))
 (via (at 30.000 33.000) (size 0.8) (drill 0.4) (layers "F.Cu" "B.Cu") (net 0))
 (via (at 45.000 42.000) (size 0.8) (drill 0.4) (layers "F.Cu" "B.Cu") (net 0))
 (via (at 10.000 33.000) (size 0.8) (drill 0.4) (layers "F.Cu" "B.Cu") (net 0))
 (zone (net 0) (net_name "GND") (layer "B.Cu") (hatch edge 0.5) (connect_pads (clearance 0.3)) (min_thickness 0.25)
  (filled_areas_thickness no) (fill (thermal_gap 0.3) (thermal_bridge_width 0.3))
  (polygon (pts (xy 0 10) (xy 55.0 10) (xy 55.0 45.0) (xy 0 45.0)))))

